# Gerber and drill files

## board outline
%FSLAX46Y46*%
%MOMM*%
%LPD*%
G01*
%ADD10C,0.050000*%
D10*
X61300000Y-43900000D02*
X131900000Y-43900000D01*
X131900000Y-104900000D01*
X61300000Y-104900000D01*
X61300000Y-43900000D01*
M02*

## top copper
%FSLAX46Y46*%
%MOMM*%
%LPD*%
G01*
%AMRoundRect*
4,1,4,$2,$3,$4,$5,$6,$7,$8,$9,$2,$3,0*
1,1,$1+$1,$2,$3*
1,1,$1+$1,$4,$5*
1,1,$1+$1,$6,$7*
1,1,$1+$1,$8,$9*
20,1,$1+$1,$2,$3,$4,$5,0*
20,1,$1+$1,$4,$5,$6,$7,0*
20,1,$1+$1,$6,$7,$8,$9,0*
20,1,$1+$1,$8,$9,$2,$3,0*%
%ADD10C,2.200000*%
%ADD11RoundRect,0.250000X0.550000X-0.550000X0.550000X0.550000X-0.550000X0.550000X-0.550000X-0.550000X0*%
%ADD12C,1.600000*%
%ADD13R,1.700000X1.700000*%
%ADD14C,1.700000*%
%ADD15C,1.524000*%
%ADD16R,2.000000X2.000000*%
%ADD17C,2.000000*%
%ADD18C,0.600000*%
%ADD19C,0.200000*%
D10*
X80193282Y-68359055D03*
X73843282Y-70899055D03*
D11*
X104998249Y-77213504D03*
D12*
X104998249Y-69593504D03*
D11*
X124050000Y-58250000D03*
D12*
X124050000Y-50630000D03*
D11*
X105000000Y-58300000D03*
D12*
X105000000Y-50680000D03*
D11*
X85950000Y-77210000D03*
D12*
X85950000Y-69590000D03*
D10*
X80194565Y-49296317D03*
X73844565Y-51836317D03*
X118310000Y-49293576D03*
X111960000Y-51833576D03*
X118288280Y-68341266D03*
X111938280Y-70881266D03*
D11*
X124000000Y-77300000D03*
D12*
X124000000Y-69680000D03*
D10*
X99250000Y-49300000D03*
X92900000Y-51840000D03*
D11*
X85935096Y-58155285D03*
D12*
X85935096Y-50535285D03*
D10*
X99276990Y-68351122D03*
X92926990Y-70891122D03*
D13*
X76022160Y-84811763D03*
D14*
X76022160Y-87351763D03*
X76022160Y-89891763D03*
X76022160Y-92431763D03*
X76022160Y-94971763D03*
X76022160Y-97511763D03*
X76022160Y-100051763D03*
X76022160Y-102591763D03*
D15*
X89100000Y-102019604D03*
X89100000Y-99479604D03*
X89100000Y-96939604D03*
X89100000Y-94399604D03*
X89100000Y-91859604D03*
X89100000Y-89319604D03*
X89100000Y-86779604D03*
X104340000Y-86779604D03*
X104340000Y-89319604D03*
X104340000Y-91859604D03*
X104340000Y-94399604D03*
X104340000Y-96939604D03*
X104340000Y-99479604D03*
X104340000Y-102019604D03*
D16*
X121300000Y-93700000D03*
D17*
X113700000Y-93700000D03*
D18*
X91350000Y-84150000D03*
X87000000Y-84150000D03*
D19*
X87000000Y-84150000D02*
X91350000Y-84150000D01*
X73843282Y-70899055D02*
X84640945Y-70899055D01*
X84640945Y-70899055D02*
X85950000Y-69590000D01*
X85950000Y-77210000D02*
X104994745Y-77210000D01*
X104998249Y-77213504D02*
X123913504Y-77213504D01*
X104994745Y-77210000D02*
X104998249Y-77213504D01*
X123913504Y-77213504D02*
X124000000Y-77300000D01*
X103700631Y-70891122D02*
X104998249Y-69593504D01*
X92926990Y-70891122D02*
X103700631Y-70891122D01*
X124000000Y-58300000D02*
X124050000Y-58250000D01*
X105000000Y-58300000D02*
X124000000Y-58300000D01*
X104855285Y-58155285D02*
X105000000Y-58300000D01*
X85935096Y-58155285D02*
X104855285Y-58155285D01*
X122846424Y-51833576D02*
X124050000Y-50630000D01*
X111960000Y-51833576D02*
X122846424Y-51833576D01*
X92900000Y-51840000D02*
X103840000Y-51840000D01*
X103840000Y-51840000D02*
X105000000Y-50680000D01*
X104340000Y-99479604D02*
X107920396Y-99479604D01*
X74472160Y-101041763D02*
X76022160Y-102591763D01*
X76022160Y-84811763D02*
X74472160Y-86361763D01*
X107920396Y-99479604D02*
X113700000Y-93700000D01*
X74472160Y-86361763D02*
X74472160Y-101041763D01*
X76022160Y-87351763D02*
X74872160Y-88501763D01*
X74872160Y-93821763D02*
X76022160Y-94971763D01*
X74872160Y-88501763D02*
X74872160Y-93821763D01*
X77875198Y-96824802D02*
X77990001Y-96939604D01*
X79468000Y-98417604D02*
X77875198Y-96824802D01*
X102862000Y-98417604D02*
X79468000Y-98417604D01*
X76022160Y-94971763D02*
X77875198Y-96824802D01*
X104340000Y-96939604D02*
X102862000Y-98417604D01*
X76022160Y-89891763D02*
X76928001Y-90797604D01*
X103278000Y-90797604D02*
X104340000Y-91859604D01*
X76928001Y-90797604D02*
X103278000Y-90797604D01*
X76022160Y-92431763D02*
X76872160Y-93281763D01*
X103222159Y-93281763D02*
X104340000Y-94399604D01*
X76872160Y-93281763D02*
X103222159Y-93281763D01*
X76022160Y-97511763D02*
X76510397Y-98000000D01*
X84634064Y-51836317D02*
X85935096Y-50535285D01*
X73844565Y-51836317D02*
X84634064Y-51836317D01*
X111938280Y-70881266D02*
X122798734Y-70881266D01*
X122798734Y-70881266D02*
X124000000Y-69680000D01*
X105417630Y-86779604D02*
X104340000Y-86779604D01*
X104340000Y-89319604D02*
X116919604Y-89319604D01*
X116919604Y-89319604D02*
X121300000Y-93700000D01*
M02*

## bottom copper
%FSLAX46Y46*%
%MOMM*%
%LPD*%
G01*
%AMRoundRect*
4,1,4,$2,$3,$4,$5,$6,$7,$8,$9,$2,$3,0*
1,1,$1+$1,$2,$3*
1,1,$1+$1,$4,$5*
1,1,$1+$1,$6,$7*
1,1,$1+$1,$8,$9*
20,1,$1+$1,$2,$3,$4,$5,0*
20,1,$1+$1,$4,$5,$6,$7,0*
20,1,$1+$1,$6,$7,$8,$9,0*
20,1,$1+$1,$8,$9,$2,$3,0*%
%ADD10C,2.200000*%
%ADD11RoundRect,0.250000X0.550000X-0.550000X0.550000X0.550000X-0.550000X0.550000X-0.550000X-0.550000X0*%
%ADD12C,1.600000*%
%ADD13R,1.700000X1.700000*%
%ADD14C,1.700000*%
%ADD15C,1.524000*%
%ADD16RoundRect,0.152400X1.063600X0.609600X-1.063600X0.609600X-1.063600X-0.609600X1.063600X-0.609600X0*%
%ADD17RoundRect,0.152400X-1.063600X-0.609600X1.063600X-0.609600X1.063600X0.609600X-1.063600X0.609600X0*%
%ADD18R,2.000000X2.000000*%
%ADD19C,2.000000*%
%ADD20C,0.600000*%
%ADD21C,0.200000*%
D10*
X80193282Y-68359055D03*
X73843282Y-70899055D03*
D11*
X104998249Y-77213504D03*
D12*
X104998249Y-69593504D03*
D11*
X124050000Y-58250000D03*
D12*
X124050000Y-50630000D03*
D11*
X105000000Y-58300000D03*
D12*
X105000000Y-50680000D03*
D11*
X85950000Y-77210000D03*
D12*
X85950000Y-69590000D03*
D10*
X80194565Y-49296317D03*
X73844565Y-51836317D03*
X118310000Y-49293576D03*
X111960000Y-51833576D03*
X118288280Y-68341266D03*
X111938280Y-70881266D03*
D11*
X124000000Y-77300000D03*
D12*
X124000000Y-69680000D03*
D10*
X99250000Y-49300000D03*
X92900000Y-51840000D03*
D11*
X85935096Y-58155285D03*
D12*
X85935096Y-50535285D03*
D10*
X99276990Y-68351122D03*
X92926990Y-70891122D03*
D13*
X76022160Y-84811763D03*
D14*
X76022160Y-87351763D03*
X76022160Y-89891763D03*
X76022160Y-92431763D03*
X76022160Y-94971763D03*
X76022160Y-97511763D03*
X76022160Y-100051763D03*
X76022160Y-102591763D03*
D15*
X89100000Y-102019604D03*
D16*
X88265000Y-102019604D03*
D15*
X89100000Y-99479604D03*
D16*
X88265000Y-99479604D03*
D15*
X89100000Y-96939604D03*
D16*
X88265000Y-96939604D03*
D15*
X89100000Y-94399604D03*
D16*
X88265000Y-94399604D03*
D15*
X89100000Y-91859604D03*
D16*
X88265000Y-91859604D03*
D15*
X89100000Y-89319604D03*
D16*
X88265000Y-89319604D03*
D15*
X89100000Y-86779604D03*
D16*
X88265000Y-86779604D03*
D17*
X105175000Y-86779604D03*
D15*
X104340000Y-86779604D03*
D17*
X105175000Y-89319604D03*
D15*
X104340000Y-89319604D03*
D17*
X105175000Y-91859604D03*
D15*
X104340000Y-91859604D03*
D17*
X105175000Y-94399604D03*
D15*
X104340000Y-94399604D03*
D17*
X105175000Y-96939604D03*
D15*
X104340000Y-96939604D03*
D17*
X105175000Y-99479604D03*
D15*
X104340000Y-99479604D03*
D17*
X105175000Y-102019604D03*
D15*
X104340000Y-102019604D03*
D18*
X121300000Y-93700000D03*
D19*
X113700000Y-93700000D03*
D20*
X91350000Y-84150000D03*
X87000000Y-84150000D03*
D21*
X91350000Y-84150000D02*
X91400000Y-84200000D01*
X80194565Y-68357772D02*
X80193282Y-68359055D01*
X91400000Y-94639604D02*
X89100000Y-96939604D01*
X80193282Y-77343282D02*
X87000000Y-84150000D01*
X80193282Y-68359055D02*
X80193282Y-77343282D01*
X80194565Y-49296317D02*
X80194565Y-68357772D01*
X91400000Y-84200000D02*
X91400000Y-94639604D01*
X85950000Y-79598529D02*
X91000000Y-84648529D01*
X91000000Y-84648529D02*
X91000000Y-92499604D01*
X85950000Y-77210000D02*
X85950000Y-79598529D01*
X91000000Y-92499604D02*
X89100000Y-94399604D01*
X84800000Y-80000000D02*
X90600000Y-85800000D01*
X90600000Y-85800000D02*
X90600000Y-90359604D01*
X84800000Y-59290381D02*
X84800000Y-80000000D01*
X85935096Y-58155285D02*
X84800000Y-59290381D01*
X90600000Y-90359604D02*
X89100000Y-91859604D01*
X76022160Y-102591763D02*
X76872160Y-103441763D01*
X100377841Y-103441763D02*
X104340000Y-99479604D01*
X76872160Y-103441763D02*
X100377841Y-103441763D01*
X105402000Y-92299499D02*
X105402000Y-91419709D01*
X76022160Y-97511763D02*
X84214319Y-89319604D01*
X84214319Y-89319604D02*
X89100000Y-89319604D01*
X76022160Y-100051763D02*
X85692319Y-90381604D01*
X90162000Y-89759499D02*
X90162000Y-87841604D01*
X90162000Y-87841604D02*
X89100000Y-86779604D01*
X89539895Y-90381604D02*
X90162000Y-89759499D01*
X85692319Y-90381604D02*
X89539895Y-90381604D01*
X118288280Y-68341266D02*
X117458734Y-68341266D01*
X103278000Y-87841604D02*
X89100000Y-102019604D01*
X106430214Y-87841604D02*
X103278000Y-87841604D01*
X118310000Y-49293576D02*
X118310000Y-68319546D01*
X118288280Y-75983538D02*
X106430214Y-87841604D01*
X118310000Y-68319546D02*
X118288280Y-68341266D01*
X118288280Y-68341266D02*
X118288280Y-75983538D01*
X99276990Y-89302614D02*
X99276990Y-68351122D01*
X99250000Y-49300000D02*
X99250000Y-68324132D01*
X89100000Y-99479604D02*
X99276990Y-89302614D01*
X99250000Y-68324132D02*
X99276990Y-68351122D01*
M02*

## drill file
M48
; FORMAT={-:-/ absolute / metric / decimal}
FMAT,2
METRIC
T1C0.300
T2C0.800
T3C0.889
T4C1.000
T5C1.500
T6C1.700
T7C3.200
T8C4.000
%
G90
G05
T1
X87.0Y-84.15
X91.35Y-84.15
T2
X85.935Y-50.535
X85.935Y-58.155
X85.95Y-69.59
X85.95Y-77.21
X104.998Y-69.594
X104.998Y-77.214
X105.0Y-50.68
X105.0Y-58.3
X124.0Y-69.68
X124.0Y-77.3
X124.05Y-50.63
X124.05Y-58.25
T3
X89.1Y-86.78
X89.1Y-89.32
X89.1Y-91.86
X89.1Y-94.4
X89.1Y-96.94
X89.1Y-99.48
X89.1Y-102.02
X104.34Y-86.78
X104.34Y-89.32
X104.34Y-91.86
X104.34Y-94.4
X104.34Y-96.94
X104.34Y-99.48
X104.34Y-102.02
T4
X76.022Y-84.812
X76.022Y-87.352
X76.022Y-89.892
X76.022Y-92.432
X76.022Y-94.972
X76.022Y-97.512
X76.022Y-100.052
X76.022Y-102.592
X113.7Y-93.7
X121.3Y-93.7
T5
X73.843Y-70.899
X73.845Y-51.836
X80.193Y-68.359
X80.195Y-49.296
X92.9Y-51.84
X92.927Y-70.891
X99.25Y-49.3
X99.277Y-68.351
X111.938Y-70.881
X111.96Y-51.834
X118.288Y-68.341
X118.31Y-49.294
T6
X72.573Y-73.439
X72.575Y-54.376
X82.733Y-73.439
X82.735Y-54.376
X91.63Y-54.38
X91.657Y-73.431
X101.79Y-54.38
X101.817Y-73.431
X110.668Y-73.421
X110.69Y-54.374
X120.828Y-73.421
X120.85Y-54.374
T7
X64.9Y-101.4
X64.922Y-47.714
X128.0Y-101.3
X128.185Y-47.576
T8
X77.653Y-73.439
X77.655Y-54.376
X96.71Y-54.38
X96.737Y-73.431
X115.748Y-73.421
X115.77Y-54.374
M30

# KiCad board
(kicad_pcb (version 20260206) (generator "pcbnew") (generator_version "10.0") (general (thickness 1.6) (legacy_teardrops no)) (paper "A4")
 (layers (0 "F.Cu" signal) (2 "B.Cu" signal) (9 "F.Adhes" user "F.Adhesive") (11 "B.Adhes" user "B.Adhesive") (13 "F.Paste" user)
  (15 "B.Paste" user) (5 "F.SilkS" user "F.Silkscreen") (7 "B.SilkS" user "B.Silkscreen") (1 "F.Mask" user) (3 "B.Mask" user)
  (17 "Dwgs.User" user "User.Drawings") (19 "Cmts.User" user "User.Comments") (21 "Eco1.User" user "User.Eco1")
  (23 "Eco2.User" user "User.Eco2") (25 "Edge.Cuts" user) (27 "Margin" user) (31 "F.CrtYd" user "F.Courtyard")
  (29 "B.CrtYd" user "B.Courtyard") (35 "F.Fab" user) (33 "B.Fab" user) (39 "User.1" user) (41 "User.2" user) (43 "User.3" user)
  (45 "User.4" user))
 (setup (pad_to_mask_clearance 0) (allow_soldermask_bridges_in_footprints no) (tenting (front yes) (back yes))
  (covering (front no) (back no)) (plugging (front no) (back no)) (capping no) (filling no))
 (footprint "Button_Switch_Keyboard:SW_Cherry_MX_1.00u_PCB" (layer "F.Cu") (at 80.193282 68.359055)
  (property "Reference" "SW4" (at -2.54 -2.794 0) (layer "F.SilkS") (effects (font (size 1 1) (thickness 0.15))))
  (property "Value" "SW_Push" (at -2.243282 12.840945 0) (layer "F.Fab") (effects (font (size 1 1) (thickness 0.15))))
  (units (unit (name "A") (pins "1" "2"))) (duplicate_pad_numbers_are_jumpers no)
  (pad "" np_thru_hole circle (at -7.62 5.08) (size 1.7 1.7) (drill 1.7) (layers "*.Cu" "*.Mask"))
  (pad "" np_thru_hole circle (at -2.54 5.08) (size 4 4) (drill 4) (layers "*.Cu" "*.Mask"))
  (pad "" np_thru_hole circle (at 2.54 5.08) (size 1.7 1.7) (drill 1.7) (layers "*.Cu" "*.Mask"))
  (pad "1" thru_hole circle (at 0 0) (size 2.2 2.2) (drill 1.5) (layers "*.Cu" "*.Mask") (remove_unused_layers no) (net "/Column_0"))
  (pad "2" thru_hole circle (at -6.35 2.54) (size 2.2 2.2) (drill 1.5) (layers "*.Cu" "*.Mask") (remove_unused_layers no) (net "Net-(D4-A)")))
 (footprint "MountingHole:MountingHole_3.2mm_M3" (layer "F.Cu") (at 64.922216 47.713994)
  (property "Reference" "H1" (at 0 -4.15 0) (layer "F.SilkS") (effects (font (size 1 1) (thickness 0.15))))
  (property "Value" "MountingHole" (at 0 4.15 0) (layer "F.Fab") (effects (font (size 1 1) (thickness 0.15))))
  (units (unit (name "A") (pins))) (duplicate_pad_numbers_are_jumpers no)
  (pad "" np_thru_hole circle (at 0 0) (size 3.2 3.2) (drill 3.2) (layers "*.Cu" "*.Mask")))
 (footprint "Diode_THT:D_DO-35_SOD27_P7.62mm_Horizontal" (layer "F.Cu") (at 104.998249 77.213504 90)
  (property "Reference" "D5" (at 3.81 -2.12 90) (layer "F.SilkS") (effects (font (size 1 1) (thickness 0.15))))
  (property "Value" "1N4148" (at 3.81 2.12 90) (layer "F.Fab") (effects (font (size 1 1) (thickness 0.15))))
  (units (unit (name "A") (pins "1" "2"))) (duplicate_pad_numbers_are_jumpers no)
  (pad "1" thru_hole roundrect (at 0 0 90) (size 1.6 1.6) (drill 0.8) (layers "*.Cu" "*.Mask") (remove_unused_layers no)
   (roundrect_rratio 0.15625) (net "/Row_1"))
  (pad "2" thru_hole circle (at 7.62 0 90) (size 1.6 1.6) (drill 0.8) (layers "*.Cu" "*.Mask") (remove_unused_layers no) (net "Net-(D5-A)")))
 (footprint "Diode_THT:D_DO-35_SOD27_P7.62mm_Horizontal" (layer "F.Cu") (at 124.05 58.25 90)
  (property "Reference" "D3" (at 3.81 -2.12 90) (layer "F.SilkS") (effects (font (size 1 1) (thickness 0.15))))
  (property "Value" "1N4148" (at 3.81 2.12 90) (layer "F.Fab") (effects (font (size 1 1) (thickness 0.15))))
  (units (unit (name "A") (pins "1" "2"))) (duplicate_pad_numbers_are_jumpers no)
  (pad "1" thru_hole roundrect (at 0 0 90) (size 1.6 1.6) (drill 0.8) (layers "*.Cu" "*.Mask") (remove_unused_layers no)
   (roundrect_rratio 0.15625) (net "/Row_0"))
  (pad "2" thru_hole circle (at 7.62 0 90) (size 1.6 1.6) (drill 0.8) (layers "*.Cu" "*.Mask") (remove_unused_layers no) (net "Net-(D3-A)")))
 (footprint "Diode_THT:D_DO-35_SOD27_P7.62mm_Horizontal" (layer "F.Cu") (at 105 58.3 90)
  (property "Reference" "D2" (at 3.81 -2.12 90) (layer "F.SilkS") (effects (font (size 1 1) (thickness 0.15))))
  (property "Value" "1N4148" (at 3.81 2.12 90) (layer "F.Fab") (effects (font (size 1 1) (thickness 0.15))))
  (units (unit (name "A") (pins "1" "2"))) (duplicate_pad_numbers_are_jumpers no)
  (pad "1" thru_hole roundrect (at 0 0 90) (size 1.6 1.6) (drill 0.8) (layers "*.Cu" "*.Mask") (remove_unused_layers no)
   (roundrect_rratio 0.15625) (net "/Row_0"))
  (pad "2" thru_hole circle (at 7.62 0 90) (size 1.6 1.6) (drill 0.8) (layers "*.Cu" "*.Mask") (remove_unused_layers no) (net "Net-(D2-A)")))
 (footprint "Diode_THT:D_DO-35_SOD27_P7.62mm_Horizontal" (layer "F.Cu") (at 85.95 77.21 90)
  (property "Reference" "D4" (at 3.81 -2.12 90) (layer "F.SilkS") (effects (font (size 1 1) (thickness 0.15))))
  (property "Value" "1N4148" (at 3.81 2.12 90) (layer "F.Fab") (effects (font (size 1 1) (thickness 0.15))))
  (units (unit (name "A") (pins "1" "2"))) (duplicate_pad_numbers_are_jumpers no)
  (pad "1" thru_hole roundrect (at 0 0 90) (size 1.6 1.6) (drill 0.8) (layers "*.Cu" "*.Mask") (remove_unused_layers no)
   (roundrect_rratio 0.15625) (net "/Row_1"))
  (pad "2" thru_hole circle (at 7.62 0 90) (size 1.6 1.6) (drill 0.8) (layers "*.Cu" "*.Mask") (remove_unused_layers no) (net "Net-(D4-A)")))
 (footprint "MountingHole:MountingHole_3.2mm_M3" (layer "F.Cu") (at 128 101.3)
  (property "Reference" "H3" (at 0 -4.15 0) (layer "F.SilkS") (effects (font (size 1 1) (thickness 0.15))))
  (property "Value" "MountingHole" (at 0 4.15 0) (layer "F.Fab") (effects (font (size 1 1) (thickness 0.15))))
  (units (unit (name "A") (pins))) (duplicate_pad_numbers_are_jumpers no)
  (pad "" np_thru_hole circle (at 0 0) (size 3.2 3.2) (drill 3.2) (layers "*.Cu" "*.Mask")))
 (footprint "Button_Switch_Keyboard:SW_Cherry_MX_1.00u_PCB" (layer "F.Cu") (at 80.194565 49.296317)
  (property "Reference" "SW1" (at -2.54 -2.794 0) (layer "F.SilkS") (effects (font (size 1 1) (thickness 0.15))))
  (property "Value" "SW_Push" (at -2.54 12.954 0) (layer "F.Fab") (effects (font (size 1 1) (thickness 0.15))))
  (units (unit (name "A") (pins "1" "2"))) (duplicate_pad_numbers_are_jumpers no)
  (pad "" np_thru_hole circle (at -7.62 5.08) (size 1.7 1.7) (drill 1.7) (layers "*.Cu" "*.Mask"))
  (pad "" np_thru_hole circle (at -2.54 5.08) (size 4 4) (drill 4) (layers "*.Cu" "*.Mask"))
  (pad "" np_thru_hole circle (at 2.54 5.08) (size 1.7 1.7) (drill 1.7) (layers "*.Cu" "*.Mask"))
  (pad "1" thru_hole circle (at 0 0) (size 2.2 2.2) (drill 1.5) (layers "*.Cu" "*.Mask") (remove_unused_layers no) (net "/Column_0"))
  (pad "2" thru_hole circle (at -6.35 2.54) (size 2.2 2.2) (drill 1.5) (layers "*.Cu" "*.Mask") (remove_unused_layers no) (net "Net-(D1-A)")))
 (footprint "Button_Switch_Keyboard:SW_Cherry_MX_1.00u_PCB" (layer "F.Cu") (at 118.31 49.293576)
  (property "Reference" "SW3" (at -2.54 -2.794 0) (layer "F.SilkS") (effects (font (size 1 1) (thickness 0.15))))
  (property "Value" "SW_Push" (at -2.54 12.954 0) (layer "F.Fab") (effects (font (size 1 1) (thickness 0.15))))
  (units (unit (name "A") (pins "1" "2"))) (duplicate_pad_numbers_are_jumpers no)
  (pad "" np_thru_hole circle (at -7.62 5.08) (size 1.7 1.7) (drill 1.7) (layers "*.Cu" "*.Mask"))
  (pad "" np_thru_hole circle (at -2.54 5.08) (size 4 4) (drill 4) (layers "*.Cu" "*.Mask"))
  (pad "" np_thru_hole circle (at 2.54 5.08) (size 1.7 1.7) (drill 1.7) (layers "*.Cu" "*.Mask"))
  (pad "1" thru_hole circle (at 0 0) (size 2.2 2.2) (drill 1.5) (layers "*.Cu" "*.Mask") (remove_unused_layers no) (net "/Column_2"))
  (pad "2" thru_hole circle (at -6.35 2.54) (size 2.2 2.2) (drill 1.5) (layers "*.Cu" "*.Mask") (remove_unused_layers no) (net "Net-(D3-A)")))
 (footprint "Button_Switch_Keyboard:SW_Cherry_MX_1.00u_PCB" (layer "F.Cu") (at 118.28828 68.341266)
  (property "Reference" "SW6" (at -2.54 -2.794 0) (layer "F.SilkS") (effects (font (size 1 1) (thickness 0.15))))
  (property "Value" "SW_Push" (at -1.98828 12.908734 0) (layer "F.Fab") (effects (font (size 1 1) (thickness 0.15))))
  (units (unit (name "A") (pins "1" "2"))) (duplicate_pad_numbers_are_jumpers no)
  (pad "" np_thru_hole circle (at -7.62 5.08) (size 1.7 1.7) (drill 1.7) (layers "*.Cu" "*.Mask"))
  (pad "" np_thru_hole circle (at -2.54 5.08) (size 4 4) (drill 4) (layers "*.Cu" "*.Mask"))
  (pad "" np_thru_hole circle (at 2.54 5.08) (size 1.7 1.7) (drill 1.7) (layers "*.Cu" "*.Mask"))
  (pad "1" thru_hole circle (at 0 0) (size 2.2 2.2) (drill 1.5) (layers "*.Cu" "*.Mask") (remove_unused_layers no) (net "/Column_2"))
  (pad "2" thru_hole circle (at -6.35 2.54) (size 2.2 2.2) (drill 1.5) (layers "*.Cu" "*.Mask") (remove_unused_layers no) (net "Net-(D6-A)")))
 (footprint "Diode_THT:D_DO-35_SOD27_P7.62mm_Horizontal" (layer "F.Cu") (at 124 77.3 90)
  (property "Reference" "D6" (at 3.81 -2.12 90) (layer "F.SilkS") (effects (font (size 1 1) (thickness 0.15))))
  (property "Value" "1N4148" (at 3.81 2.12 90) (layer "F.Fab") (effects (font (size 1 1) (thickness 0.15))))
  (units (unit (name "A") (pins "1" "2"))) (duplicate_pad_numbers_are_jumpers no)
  (pad "1" thru_hole roundrect (at 0 0 90) (size 1.6 1.6) (drill 0.8) (layers "*.Cu" "*.Mask") (remove_unused_layers no)
   (roundrect_rratio 0.15625) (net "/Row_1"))
  (pad "2" thru_hole circle (at 7.62 0 90) (size 1.6 1.6) (drill 0.8) (layers "*.Cu" "*.Mask") (remove_unused_layers no) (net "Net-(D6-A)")))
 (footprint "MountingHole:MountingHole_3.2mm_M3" (layer "F.Cu") (at 64.9 101.4)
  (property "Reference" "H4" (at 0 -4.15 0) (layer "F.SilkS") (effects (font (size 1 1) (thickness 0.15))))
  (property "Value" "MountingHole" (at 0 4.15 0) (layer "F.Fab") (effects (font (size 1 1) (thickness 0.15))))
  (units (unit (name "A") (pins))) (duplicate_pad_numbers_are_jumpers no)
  (pad "" np_thru_hole circle (at 0 0) (size 3.2 3.2) (drill 3.2) (layers "*.Cu" "*.Mask")))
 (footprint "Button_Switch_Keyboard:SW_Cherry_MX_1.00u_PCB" (layer "F.Cu") (at 99.25 49.3)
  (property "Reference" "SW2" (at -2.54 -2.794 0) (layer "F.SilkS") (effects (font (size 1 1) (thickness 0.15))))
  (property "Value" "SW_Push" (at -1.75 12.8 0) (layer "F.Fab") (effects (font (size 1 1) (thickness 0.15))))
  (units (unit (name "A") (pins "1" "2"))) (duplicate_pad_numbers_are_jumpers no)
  (pad "" np_thru_hole circle (at -7.62 5.08) (size 1.7 1.7) (drill 1.7) (layers "*.Cu" "*.Mask"))
  (pad "" np_thru_hole circle (at -2.54 5.08) (size 4 4) (drill 4) (layers "*.Cu" "*.Mask"))
  (pad "" np_thru_hole circle (at 2.54 5.08) (size 1.7 1.7) (drill 1.7) (layers "*.Cu" "*.Mask"))
  (pad "1" thru_hole circle (at 0 0) (size 2.2 2.2) (drill 1.5) (layers "*.Cu" "*.Mask") (remove_unused_layers no) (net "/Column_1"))
  (pad "2" thru_hole circle (at -6.35 2.54) (size 2.2 2.2) (drill 1.5) (layers "*.Cu" "*.Mask") (remove_unused_layers no) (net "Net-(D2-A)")))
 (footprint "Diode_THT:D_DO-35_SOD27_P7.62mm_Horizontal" (layer "F.Cu") (at 85.935096 58.155285 90)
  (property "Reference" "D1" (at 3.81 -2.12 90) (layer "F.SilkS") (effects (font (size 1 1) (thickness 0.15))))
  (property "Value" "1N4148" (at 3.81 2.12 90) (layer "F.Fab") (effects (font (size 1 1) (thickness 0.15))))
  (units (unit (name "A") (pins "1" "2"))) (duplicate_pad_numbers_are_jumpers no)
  (pad "1" thru_hole roundrect (at 0 0 90) (size 1.6 1.6) (drill 0.8) (layers "*.Cu" "*.Mask") (remove_unused_layers no)
   (roundrect_rratio 0.15625) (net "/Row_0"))
  (pad "2" thru_hole circle (at 7.62 0 90) (size 1.6 1.6) (drill 0.8) (layers "*.Cu" "*.Mask") (remove_unused_layers no) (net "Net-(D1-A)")))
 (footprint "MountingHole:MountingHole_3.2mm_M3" (layer "F.Cu") (at 128.184744 47.576052)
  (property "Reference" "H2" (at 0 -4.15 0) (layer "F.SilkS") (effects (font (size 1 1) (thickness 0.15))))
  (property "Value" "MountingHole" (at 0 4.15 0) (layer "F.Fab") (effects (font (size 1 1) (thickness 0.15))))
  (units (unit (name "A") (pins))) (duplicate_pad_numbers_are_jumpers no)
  (pad "" np_thru_hole circle (at 0 0) (size 3.2 3.2) (drill 3.2) (layers "*.Cu" "*.Mask")))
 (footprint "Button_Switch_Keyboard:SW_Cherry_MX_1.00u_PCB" (layer "F.Cu") (at 99.27699 68.351122)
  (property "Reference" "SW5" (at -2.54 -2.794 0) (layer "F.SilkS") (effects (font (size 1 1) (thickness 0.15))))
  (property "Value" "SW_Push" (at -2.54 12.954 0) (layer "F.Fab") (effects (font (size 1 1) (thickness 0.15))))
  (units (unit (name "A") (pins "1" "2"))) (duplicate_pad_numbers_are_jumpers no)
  (pad "" np_thru_hole circle (at -7.62 5.08) (size 1.7 1.7) (drill 1.7) (layers "*.Cu" "*.Mask"))
  (pad "" np_thru_hole circle (at -2.54 5.08) (size 4 4) (drill 4) (layers "*.Cu" "*.Mask"))
  (pad "" np_thru_hole circle (at 2.54 5.08) (size 1.7 1.7) (drill 1.7) (layers "*.Cu" "*.Mask"))
  (pad "1" thru_hole circle (at 0 0) (size 2.2 2.2) (drill 1.5) (layers "*.Cu" "*.Mask") (remove_unused_layers no) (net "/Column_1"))
  (pad "2" thru_hole circle (at -6.35 2.54) (size 2.2 2.2) (drill 1.5) (layers "*.Cu" "*.Mask") (remove_unused_layers no) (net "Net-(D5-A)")))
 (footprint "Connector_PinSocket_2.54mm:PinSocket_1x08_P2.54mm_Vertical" (layer "B.Cu") (at 76.02216 84.811763 180)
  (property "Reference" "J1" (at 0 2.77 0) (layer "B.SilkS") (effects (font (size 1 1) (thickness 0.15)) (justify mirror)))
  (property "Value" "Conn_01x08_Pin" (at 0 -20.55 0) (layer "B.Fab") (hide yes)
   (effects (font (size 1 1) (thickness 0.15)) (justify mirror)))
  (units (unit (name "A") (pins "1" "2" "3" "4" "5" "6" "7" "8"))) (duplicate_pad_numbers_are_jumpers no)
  (pad "1" thru_hole rect (at 0 0 180) (size 1.7 1.7) (drill 1) (layers "*.Cu" "*.Mask") (remove_unused_layers no) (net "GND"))
  (pad "2" thru_hole circle (at 0 -2.54 180) (size 1.7 1.7) (drill 1) (layers "*.Cu" "*.Mask") (remove_unused_layers no) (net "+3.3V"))
  (pad "3" thru_hole circle (at 0 -5.08 180) (size 1.7 1.7) (drill 1) (layers "*.Cu" "*.Mask") (remove_unused_layers no) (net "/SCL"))
  (pad "4" thru_hole circle (at 0 -7.62 180) (size 1.7 1.7) (drill 1) (layers "*.Cu" "*.Mask") (remove_unused_layers no) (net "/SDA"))
  (pad "5" thru_hole circle (at 0 -10.16 180) (size 1.7 1.7) (drill 1) (layers "*.Cu" "*.Mask") (remove_unused_layers no) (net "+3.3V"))
  (pad "6" thru_hole circle (at 0 -12.7 180) (size 1.7 1.7) (drill 1) (layers "*.Cu" "*.Mask") (remove_unused_layers no) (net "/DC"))
  (pad "7" thru_hole circle (at 0 -15.24 180) (size 1.7 1.7) (drill 1) (layers "*.Cu" "*.Mask") (remove_unused_layers no) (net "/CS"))
  (pad "8" thru_hole circle (at 0 -17.78 180) (size 1.7 1.7) (drill 1) (layers "*.Cu" "*.Mask") (remove_unused_layers no) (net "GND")))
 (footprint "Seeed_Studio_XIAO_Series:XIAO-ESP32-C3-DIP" (layer "B.Cu") (at 96.72 94.399604 -90)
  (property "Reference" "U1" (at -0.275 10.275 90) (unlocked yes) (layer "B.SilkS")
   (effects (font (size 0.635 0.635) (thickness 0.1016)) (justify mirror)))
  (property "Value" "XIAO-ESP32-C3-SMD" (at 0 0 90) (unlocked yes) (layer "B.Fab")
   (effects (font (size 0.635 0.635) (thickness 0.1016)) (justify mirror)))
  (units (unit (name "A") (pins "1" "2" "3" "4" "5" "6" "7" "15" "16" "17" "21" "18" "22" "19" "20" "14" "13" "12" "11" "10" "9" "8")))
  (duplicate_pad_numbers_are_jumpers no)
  (pad "1" thru_hole circle (at 7.62 7.62 180) (size 1.524 1.524) (drill 0.889) (layers "*.Cu" "*.Mask") (remove_unused_layers no)
   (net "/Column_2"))
  (pad "1" smd roundrect (at 7.62 8.455 180) (size 2.432 1.524) (layers "B.Cu" "B.Mask") (roundrect_rratio 0.1) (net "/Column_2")
   (thermal_bridge_angle 45))
  (pad "2" thru_hole circle (at 5.08 7.62 180) (size 1.524 1.524) (drill 0.889) (layers "*.Cu" "*.Mask") (remove_unused_layers no)
   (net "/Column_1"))
  (pad "2" smd roundrect (at 5.08 8.455 180) (size 2.432 1.524) (layers "B.Cu" "B.Mask") (roundrect_rratio 0.1) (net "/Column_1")
   (thermal_bridge_angle 45))
  (pad "3" thru_hole circle (at 2.54 7.62 180) (size 1.524 1.524) (drill 0.889) (layers "*.Cu" "*.Mask") (remove_unused_layers no)
   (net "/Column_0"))
  (pad "3" smd roundrect (at 2.54 8.455 180) (size 2.432 1.524) (layers "B.Cu" "B.Mask") (roundrect_rratio 0.1) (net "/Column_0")
   (thermal_bridge_angle 45))
  (pad "4" thru_hole circle (at 0 7.62 180) (size 1.524 1.524) (drill 0.889) (layers "*.Cu" "*.Mask") (remove_unused_layers no)
   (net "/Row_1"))
  (pad "4" smd roundrect (at 0 8.455 180) (size 2.432 1.524) (layers "B.Cu" "B.Mask") (roundrect_rratio 0.1) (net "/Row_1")
   (thermal_bridge_angle 45))
  (pad "5" thru_hole circle (at -2.54 7.62 180) (size 1.524 1.524) (drill 0.889) (layers "*.Cu" "*.Mask") (remove_unused_layers no)
   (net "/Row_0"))
  (pad "5" smd roundrect (at -2.54 8.455 180) (size 2.432 1.524) (layers "B.Cu" "B.Mask") (roundrect_rratio 0.1) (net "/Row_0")
   (thermal_bridge_angle 45))
  (pad "6" thru_hole circle (at -5.08 7.62 180) (size 1.524 1.524) (drill 0.889) (layers "*.Cu" "*.Mask") (remove_unused_layers no)
   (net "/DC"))
  (pad "6" smd roundrect (at -5.08 8.455 180) (size 2.432 1.524) (layers "B.Cu" "B.Mask") (roundrect_rratio 0.1) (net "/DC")
   (thermal_bridge_angle 45))
  (pad "7" thru_hole circle (at -7.62 7.62 180) (size 1.524 1.524) (drill 0.889) (layers "*.Cu" "*.Mask") (remove_unused_layers no)
   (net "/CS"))
  (pad "7" smd roundrect (at -7.62 8.455 180) (size 2.432 1.524) (layers "B.Cu" "B.Mask") (roundrect_rratio 0.1) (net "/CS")
   (thermal_bridge_angle 45))
  (pad "8" smd roundrect (at -7.62 -8.455) (size 2.432 1.524) (layers "B.Cu" "B.Mask") (roundrect_rratio 0.1)
   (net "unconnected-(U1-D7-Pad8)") (thermal_bridge_angle 45))
  (pad "8" thru_hole circle (at -7.62 -7.62) (size 1.524 1.524) (drill 0.889) (layers "*.Cu" "*.Mask") (remove_unused_layers no)
   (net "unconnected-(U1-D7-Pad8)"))
  (pad "9" smd roundrect (at -5.08 -8.455) (size 2.432 1.524) (layers "B.Cu" "B.Mask") (roundrect_rratio 0.1) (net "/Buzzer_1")
   (thermal_bridge_angle 45))
  (pad "9" thru_hole circle (at -5.08 -7.62) (size 1.524 1.524) (drill 0.889) (layers "*.Cu" "*.Mask") (remove_unused_layers no)
   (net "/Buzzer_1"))
  (pad "10" smd roundrect (at -2.54 -8.455) (size 2.432 1.524) (layers "B.Cu" "B.Mask") (roundrect_rratio 0.1) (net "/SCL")
   (thermal_bridge_angle 45))
  (pad "10" thru_hole circle (at -2.54 -7.62) (size 1.524 1.524) (drill 0.889) (layers "*.Cu" "*.Mask") (remove_unused_layers no)
   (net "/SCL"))
  (pad "11" smd roundrect (at 0 -8.455) (size 2.432 1.524) (layers "B.Cu" "B.Mask") (roundrect_rratio 0.1) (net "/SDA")
   (thermal_bridge_angle 45))
  (pad "11" thru_hole circle (at 0 -7.62) (size 1.524 1.524) (drill 0.889) (layers "*.Cu" "*.Mask") (remove_unused_layers no) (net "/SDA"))
  (pad "12" smd roundrect (at 2.54 -8.455) (size 2.432 1.524) (layers "B.Cu" "B.Mask") (roundrect_rratio 0.1) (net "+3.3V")
   (thermal_bridge_angle 45))
  (pad "12" thru_hole circle (at 2.54 -7.62) (size 1.524 1.524) (drill 0.889) (layers "*.Cu" "*.Mask") (remove_unused_layers no)
   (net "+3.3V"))
  (pad "13" smd roundrect (at 5.08 -8.455) (size 2.432 1.524) (layers "B.Cu" "B.Mask") (roundrect_rratio 0.1) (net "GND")
   (thermal_bridge_angle 45))
  (pad "13" thru_hole circle (at 5.08 -7.62) (size 1.524 1.524) (drill 0.889) (layers "*.Cu" "*.Mask") (remove_unused_layers no) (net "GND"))
  (pad "14" smd roundrect (at 7.62 -8.455) (size 2.432 1.524) (layers "B.Cu" "B.Mask") (roundrect_rratio 0.1)
   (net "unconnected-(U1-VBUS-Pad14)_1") (thermal_bridge_angle 45))
  (pad "14" thru_hole circle (at 7.62 -7.62) (size 1.524 1.524) (drill 0.889) (layers "*.Cu" "*.Mask") (remove_unused_layers no)
   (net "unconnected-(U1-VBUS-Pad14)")))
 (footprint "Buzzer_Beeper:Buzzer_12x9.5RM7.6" (layer "B.Cu") (at 121.3 93.7 180)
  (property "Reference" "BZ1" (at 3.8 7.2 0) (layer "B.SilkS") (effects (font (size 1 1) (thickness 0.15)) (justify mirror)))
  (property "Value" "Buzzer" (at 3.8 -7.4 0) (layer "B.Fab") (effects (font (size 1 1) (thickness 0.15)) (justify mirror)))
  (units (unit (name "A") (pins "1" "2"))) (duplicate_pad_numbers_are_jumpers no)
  (pad "1" thru_hole rect (at 0 0 180) (size 2 2) (drill 1) (layers "*.Cu" "*.Mask") (remove_unused_layers no) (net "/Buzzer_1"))
  (pad "2" thru_hole circle (at 7.6 0 180) (size 2 2) (drill 1) (layers "*.Cu" "*.Mask") (remove_unused_layers no) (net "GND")))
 (gr_rect (start 61.3 43.9) (end 131.9 104.9) (stroke (width 0.05) (type default)) (fill no) (layer "Edge.Cuts"))
 (segment (start 87 84.15) (end 91.35 84.15) (width 0.2) (layer "F.Cu") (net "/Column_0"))
 (via (at 91.35 84.15) (size 0.6) (drill 0.3) (layers "F.Cu" "B.Cu") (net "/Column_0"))
 (via (at 87 84.15) (size 0.6) (drill 0.3) (layers "F.Cu" "B.Cu") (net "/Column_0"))
 (segment (start 91.35 84.15) (end 91.4 84.2) (width 0.2) (layer "B.Cu") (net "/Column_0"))
 (segment (start 80.194565 68.357772) (end 80.193282 68.359055) (width 0.2) (layer "B.Cu") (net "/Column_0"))
 (segment (start 91.4 94.639604) (end 89.1 96.939604) (width 0.2) (layer "B.Cu") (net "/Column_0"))
 (segment (start 80.193282 77.343282) (end 87 84.15) (width 0.2) (layer "B.Cu") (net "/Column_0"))
 (segment (start 80.193282 68.359055) (end 80.193282 77.343282) (width 0.2) (layer "B.Cu") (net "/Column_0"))
 (segment (start 80.194565 49.296317) (end 80.194565 68.357772) (width 0.2) (layer "B.Cu") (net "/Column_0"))
 (segment (start 91.4 84.2) (end 91.4 94.639604) (width 0.2) (layer "B.Cu") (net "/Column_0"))
 (segment (start 73.843282 70.899055) (end 84.640945 70.899055) (width 0.2) (layer "F.Cu") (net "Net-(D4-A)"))
 (segment (start 84.640945 70.899055) (end 85.95 69.59) (width 0.2) (layer "F.Cu") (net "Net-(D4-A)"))
 (segment (start 85.95 77.21) (end 104.994745 77.21) (width 0.2) (layer "F.Cu") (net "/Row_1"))
 (segment (start 104.998249 77.213504) (end 123.913504 77.213504) (width 0.2) (layer "F.Cu") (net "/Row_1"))
 (segment (start 104.994745 77.21) (end 104.998249 77.213504) (width 0.2) (layer "F.Cu") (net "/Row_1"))
 (segment (start 123.913504 77.213504) (end 124 77.3) (width 0.2) (layer "F.Cu") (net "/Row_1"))
 (segment (start 85.95 79.598529) (end 91 84.648529) (width 0.2) (layer "B.Cu") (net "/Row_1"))
 (segment (start 91 84.648529) (end 91 92.499604) (width 0.2) (layer "B.Cu") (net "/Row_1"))
 (segment (start 85.95 77.21) (end 85.95 79.598529) (width 0.2) (layer "B.Cu") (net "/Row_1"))
 (segment (start 91 92.499604) (end 89.1 94.399604) (width 0.2) (layer "B.Cu") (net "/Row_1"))
 (segment (start 103.700631 70.891122) (end 104.998249 69.593504) (width 0.2) (layer "F.Cu") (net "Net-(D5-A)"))
 (segment (start 92.92699 70.891122) (end 103.700631 70.891122) (width 0.2) (layer "F.Cu") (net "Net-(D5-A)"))
 (segment (start 124 58.3) (end 124.05 58.25) (width 0.2) (layer "F.Cu") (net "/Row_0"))
 (segment (start 105 58.3) (end 124 58.3) (width 0.2) (layer "F.Cu") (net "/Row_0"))
 (segment (start 104.855285 58.155285) (end 105 58.3) (width 0.2) (layer "F.Cu") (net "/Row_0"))
 (segment (start 85.935096 58.155285) (end 104.855285 58.155285) (width 0.2) (layer "F.Cu") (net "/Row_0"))
 (segment (start 84.8 80) (end 90.6 85.8) (width 0.2) (layer "B.Cu") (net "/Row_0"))
 (segment (start 90.6 85.8) (end 90.6 90.359604) (width 0.2) (layer "B.Cu") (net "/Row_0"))
 (segment (start 84.8 59.290381) (end 84.8 80) (width 0.2) (layer "B.Cu") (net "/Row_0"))
 (segment (start 85.935096 58.155285) (end 84.8 59.290381) (width 0.2) (layer "B.Cu") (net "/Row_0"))
 (segment (start 90.6 90.359604) (end 89.1 91.859604) (width 0.2) (layer "B.Cu") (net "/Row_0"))
 (segment (start 122.846424 51.833576) (end 124.05 50.63) (width 0.2) (layer "F.Cu") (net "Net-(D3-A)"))
 (segment (start 111.96 51.833576) (end 122.846424 51.833576) (width 0.2) (layer "F.Cu") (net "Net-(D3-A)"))
 (segment (start 92.9 51.84) (end 103.84 51.84) (width 0.2) (layer "F.Cu") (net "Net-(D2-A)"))
 (segment (start 103.84 51.84) (end 105 50.68) (width 0.2) (layer "F.Cu") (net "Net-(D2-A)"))
 (segment (start 104.34 99.479604) (end 107.920396 99.479604) (width 0.2) (layer "F.Cu") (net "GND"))
 (segment (start 74.47216 101.041763) (end 76.02216 102.591763) (width 0.2) (layer "F.Cu") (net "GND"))
 (segment (start 76.02216 84.811763) (end 74.47216 86.361763) (width 0.2) (layer "F.Cu") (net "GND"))
 (segment (start 107.920396 99.479604) (end 113.7 93.7) (width 0.2) (layer "F.Cu") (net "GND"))
 (segment (start 74.47216 86.361763) (end 74.47216 101.041763) (width 0.2) (layer "F.Cu") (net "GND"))
 (segment (start 76.02216 102.591763) (end 76.87216 103.441763) (width 0.2) (layer "B.Cu") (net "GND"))
 (segment (start 100.377841 103.441763) (end 104.34 99.479604) (width 0.2) (layer "B.Cu") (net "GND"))
 (segment (start 76.87216 103.441763) (end 100.377841 103.441763) (width 0.2) (layer "B.Cu") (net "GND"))
 (segment (start 76.02216 87.351763) (end 74.87216 88.501763) (width 0.2) (layer "F.Cu") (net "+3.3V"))
 (segment (start 74.87216 93.821763) (end 76.02216 94.971763) (width 0.2) (layer "F.Cu") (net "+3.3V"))
 (segment (start 74.87216 88.501763) (end 74.87216 93.821763) (width 0.2) (layer "F.Cu") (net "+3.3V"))
 (segment (start 77.875198 96.824802) (end 77.990001 96.939604) (width 0.2) (layer "F.Cu") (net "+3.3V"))
 (segment (start 79.468 98.417604) (end 77.875198 96.824802) (width 0.2) (layer "F.Cu") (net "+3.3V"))
 (segment (start 102.862 98.417604) (end 79.468 98.417604) (width 0.2) (layer "F.Cu") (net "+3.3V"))
 (segment (start 76.02216 94.971763) (end 77.875198 96.824802) (width 0.2) (layer "F.Cu") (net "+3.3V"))
 (segment (start 104.34 96.939604) (end 102.862 98.417604) (width 0.2) (layer "F.Cu") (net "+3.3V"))
 (segment (start 76.02216 89.891763) (end 76.928001 90.797604) (width 0.2) (layer "F.Cu") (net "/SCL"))
 (segment (start 103.278 90.797604) (end 104.34 91.859604) (width 0.2) (layer "F.Cu") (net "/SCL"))
 (segment (start 76.928001 90.797604) (end 103.278 90.797604) (width 0.2) (layer "F.Cu") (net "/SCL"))
 (segment (start 105.402 92.299499) (end 105.402 91.419709) (width 0.2) (layer "B.Cu") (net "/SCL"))
 (segment (start 76.02216 92.431763) (end 76.87216 93.281763) (width 0.2) (layer "F.Cu") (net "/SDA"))
 (segment (start 103.222159 93.281763) (end 104.34 94.399604) (width 0.2) (layer "F.Cu") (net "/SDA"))
 (segment (start 76.87216 93.281763) (end 103.222159 93.281763) (width 0.2) (layer "F.Cu") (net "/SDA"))
 (segment (start 76.02216 97.511763) (end 76.510397 98) (width 0.2) (layer "F.Cu") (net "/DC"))
 (segment (start 76.02216 97.511763) (end 84.214319 89.319604) (width 0.2) (layer "B.Cu") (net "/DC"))
 (segment (start 84.214319 89.319604) (end 89.1 89.319604) (width 0.2) (layer "B.Cu") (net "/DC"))
 (segment (start 76.02216 100.051763) (end 85.692319 90.381604) (width 0.2) (layer "B.Cu") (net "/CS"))
 (segment (start 90.162 89.759499) (end 90.162 87.841604) (width 0.2) (layer "B.Cu") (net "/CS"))
 (segment (start 90.162 87.841604) (end 89.1 86.779604) (width 0.2) (layer "B.Cu") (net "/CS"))
 (segment (start 89.539895 90.381604) (end 90.162 89.759499) (width 0.2) (layer "B.Cu") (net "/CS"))
 (segment (start 85.692319 90.381604) (end 89.539895 90.381604) (width 0.2) (layer "B.Cu") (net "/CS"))
 (segment (start 84.634064 51.836317) (end 85.935096 50.535285) (width 0.2) (layer "F.Cu") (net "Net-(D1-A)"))
 (segment (start 73.844565 51.836317) (end 84.634064 51.836317) (width 0.2) (layer "F.Cu") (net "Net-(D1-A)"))
 (segment (start 118.28828 68.341266) (end 117.458734 68.341266) (width 0.2) (layer "B.Cu") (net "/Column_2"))
 (segment (start 103.278 87.841604) (end 89.1 102.019604) (width 0.2) (layer "B.Cu") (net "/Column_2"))
 (segment (start 106.430214 87.841604) (end 103.278 87.841604) (width 0.2) (layer "B.Cu") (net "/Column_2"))
 (segment (start 118.31 49.293576) (end 118.31 68.319546) (width 0.2) (layer "B.Cu") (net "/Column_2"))
 (segment (start 118.28828 75.983538) (end 106.430214 87.841604) (width 0.2) (layer "B.Cu") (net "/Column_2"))
 (segment (start 118.31 68.319546) (end 118.28828 68.341266) (width 0.2) (layer "B.Cu") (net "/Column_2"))
 (segment (start 118.28828 68.341266) (end 118.28828 75.983538) (width 0.2) (layer "B.Cu") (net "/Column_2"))
 (segment (start 111.93828 70.881266) (end 122.798734 70.881266) (width 0.2) (layer "F.Cu") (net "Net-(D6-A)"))
 (segment (start 122.798734 70.881266) (end 124 69.68) (width 0.2) (layer "F.Cu") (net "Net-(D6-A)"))
 (segment (start 99.27699 89.302614) (end 99.27699 68.351122) (width 0.2) (layer "B.Cu") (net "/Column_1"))
 (segment (start 99.25 49.3) (end 99.25 68.324132) (width 0.2) (layer "B.Cu") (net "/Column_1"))
 (segment (start 89.1 99.479604) (end 99.27699 89.302614) (width 0.2) (layer "B.Cu") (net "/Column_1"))
 (segment (start 99.25 68.324132) (end 99.27699 68.351122) (width 0.2) (layer "B.Cu") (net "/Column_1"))
 (segment (start 105.41763 86.779604) (end 104.34 86.779604) (width 0.2) (layer "F.Cu") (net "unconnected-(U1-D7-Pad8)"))
 (segment (start 104.34 89.319604) (end 116.919604 89.319604) (width 0.2) (layer "F.Cu") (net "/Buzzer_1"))
 (segment (start 116.919604 89.319604) (end 121.3 93.7) (width 0.2) (layer "F.Cu") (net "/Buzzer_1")))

